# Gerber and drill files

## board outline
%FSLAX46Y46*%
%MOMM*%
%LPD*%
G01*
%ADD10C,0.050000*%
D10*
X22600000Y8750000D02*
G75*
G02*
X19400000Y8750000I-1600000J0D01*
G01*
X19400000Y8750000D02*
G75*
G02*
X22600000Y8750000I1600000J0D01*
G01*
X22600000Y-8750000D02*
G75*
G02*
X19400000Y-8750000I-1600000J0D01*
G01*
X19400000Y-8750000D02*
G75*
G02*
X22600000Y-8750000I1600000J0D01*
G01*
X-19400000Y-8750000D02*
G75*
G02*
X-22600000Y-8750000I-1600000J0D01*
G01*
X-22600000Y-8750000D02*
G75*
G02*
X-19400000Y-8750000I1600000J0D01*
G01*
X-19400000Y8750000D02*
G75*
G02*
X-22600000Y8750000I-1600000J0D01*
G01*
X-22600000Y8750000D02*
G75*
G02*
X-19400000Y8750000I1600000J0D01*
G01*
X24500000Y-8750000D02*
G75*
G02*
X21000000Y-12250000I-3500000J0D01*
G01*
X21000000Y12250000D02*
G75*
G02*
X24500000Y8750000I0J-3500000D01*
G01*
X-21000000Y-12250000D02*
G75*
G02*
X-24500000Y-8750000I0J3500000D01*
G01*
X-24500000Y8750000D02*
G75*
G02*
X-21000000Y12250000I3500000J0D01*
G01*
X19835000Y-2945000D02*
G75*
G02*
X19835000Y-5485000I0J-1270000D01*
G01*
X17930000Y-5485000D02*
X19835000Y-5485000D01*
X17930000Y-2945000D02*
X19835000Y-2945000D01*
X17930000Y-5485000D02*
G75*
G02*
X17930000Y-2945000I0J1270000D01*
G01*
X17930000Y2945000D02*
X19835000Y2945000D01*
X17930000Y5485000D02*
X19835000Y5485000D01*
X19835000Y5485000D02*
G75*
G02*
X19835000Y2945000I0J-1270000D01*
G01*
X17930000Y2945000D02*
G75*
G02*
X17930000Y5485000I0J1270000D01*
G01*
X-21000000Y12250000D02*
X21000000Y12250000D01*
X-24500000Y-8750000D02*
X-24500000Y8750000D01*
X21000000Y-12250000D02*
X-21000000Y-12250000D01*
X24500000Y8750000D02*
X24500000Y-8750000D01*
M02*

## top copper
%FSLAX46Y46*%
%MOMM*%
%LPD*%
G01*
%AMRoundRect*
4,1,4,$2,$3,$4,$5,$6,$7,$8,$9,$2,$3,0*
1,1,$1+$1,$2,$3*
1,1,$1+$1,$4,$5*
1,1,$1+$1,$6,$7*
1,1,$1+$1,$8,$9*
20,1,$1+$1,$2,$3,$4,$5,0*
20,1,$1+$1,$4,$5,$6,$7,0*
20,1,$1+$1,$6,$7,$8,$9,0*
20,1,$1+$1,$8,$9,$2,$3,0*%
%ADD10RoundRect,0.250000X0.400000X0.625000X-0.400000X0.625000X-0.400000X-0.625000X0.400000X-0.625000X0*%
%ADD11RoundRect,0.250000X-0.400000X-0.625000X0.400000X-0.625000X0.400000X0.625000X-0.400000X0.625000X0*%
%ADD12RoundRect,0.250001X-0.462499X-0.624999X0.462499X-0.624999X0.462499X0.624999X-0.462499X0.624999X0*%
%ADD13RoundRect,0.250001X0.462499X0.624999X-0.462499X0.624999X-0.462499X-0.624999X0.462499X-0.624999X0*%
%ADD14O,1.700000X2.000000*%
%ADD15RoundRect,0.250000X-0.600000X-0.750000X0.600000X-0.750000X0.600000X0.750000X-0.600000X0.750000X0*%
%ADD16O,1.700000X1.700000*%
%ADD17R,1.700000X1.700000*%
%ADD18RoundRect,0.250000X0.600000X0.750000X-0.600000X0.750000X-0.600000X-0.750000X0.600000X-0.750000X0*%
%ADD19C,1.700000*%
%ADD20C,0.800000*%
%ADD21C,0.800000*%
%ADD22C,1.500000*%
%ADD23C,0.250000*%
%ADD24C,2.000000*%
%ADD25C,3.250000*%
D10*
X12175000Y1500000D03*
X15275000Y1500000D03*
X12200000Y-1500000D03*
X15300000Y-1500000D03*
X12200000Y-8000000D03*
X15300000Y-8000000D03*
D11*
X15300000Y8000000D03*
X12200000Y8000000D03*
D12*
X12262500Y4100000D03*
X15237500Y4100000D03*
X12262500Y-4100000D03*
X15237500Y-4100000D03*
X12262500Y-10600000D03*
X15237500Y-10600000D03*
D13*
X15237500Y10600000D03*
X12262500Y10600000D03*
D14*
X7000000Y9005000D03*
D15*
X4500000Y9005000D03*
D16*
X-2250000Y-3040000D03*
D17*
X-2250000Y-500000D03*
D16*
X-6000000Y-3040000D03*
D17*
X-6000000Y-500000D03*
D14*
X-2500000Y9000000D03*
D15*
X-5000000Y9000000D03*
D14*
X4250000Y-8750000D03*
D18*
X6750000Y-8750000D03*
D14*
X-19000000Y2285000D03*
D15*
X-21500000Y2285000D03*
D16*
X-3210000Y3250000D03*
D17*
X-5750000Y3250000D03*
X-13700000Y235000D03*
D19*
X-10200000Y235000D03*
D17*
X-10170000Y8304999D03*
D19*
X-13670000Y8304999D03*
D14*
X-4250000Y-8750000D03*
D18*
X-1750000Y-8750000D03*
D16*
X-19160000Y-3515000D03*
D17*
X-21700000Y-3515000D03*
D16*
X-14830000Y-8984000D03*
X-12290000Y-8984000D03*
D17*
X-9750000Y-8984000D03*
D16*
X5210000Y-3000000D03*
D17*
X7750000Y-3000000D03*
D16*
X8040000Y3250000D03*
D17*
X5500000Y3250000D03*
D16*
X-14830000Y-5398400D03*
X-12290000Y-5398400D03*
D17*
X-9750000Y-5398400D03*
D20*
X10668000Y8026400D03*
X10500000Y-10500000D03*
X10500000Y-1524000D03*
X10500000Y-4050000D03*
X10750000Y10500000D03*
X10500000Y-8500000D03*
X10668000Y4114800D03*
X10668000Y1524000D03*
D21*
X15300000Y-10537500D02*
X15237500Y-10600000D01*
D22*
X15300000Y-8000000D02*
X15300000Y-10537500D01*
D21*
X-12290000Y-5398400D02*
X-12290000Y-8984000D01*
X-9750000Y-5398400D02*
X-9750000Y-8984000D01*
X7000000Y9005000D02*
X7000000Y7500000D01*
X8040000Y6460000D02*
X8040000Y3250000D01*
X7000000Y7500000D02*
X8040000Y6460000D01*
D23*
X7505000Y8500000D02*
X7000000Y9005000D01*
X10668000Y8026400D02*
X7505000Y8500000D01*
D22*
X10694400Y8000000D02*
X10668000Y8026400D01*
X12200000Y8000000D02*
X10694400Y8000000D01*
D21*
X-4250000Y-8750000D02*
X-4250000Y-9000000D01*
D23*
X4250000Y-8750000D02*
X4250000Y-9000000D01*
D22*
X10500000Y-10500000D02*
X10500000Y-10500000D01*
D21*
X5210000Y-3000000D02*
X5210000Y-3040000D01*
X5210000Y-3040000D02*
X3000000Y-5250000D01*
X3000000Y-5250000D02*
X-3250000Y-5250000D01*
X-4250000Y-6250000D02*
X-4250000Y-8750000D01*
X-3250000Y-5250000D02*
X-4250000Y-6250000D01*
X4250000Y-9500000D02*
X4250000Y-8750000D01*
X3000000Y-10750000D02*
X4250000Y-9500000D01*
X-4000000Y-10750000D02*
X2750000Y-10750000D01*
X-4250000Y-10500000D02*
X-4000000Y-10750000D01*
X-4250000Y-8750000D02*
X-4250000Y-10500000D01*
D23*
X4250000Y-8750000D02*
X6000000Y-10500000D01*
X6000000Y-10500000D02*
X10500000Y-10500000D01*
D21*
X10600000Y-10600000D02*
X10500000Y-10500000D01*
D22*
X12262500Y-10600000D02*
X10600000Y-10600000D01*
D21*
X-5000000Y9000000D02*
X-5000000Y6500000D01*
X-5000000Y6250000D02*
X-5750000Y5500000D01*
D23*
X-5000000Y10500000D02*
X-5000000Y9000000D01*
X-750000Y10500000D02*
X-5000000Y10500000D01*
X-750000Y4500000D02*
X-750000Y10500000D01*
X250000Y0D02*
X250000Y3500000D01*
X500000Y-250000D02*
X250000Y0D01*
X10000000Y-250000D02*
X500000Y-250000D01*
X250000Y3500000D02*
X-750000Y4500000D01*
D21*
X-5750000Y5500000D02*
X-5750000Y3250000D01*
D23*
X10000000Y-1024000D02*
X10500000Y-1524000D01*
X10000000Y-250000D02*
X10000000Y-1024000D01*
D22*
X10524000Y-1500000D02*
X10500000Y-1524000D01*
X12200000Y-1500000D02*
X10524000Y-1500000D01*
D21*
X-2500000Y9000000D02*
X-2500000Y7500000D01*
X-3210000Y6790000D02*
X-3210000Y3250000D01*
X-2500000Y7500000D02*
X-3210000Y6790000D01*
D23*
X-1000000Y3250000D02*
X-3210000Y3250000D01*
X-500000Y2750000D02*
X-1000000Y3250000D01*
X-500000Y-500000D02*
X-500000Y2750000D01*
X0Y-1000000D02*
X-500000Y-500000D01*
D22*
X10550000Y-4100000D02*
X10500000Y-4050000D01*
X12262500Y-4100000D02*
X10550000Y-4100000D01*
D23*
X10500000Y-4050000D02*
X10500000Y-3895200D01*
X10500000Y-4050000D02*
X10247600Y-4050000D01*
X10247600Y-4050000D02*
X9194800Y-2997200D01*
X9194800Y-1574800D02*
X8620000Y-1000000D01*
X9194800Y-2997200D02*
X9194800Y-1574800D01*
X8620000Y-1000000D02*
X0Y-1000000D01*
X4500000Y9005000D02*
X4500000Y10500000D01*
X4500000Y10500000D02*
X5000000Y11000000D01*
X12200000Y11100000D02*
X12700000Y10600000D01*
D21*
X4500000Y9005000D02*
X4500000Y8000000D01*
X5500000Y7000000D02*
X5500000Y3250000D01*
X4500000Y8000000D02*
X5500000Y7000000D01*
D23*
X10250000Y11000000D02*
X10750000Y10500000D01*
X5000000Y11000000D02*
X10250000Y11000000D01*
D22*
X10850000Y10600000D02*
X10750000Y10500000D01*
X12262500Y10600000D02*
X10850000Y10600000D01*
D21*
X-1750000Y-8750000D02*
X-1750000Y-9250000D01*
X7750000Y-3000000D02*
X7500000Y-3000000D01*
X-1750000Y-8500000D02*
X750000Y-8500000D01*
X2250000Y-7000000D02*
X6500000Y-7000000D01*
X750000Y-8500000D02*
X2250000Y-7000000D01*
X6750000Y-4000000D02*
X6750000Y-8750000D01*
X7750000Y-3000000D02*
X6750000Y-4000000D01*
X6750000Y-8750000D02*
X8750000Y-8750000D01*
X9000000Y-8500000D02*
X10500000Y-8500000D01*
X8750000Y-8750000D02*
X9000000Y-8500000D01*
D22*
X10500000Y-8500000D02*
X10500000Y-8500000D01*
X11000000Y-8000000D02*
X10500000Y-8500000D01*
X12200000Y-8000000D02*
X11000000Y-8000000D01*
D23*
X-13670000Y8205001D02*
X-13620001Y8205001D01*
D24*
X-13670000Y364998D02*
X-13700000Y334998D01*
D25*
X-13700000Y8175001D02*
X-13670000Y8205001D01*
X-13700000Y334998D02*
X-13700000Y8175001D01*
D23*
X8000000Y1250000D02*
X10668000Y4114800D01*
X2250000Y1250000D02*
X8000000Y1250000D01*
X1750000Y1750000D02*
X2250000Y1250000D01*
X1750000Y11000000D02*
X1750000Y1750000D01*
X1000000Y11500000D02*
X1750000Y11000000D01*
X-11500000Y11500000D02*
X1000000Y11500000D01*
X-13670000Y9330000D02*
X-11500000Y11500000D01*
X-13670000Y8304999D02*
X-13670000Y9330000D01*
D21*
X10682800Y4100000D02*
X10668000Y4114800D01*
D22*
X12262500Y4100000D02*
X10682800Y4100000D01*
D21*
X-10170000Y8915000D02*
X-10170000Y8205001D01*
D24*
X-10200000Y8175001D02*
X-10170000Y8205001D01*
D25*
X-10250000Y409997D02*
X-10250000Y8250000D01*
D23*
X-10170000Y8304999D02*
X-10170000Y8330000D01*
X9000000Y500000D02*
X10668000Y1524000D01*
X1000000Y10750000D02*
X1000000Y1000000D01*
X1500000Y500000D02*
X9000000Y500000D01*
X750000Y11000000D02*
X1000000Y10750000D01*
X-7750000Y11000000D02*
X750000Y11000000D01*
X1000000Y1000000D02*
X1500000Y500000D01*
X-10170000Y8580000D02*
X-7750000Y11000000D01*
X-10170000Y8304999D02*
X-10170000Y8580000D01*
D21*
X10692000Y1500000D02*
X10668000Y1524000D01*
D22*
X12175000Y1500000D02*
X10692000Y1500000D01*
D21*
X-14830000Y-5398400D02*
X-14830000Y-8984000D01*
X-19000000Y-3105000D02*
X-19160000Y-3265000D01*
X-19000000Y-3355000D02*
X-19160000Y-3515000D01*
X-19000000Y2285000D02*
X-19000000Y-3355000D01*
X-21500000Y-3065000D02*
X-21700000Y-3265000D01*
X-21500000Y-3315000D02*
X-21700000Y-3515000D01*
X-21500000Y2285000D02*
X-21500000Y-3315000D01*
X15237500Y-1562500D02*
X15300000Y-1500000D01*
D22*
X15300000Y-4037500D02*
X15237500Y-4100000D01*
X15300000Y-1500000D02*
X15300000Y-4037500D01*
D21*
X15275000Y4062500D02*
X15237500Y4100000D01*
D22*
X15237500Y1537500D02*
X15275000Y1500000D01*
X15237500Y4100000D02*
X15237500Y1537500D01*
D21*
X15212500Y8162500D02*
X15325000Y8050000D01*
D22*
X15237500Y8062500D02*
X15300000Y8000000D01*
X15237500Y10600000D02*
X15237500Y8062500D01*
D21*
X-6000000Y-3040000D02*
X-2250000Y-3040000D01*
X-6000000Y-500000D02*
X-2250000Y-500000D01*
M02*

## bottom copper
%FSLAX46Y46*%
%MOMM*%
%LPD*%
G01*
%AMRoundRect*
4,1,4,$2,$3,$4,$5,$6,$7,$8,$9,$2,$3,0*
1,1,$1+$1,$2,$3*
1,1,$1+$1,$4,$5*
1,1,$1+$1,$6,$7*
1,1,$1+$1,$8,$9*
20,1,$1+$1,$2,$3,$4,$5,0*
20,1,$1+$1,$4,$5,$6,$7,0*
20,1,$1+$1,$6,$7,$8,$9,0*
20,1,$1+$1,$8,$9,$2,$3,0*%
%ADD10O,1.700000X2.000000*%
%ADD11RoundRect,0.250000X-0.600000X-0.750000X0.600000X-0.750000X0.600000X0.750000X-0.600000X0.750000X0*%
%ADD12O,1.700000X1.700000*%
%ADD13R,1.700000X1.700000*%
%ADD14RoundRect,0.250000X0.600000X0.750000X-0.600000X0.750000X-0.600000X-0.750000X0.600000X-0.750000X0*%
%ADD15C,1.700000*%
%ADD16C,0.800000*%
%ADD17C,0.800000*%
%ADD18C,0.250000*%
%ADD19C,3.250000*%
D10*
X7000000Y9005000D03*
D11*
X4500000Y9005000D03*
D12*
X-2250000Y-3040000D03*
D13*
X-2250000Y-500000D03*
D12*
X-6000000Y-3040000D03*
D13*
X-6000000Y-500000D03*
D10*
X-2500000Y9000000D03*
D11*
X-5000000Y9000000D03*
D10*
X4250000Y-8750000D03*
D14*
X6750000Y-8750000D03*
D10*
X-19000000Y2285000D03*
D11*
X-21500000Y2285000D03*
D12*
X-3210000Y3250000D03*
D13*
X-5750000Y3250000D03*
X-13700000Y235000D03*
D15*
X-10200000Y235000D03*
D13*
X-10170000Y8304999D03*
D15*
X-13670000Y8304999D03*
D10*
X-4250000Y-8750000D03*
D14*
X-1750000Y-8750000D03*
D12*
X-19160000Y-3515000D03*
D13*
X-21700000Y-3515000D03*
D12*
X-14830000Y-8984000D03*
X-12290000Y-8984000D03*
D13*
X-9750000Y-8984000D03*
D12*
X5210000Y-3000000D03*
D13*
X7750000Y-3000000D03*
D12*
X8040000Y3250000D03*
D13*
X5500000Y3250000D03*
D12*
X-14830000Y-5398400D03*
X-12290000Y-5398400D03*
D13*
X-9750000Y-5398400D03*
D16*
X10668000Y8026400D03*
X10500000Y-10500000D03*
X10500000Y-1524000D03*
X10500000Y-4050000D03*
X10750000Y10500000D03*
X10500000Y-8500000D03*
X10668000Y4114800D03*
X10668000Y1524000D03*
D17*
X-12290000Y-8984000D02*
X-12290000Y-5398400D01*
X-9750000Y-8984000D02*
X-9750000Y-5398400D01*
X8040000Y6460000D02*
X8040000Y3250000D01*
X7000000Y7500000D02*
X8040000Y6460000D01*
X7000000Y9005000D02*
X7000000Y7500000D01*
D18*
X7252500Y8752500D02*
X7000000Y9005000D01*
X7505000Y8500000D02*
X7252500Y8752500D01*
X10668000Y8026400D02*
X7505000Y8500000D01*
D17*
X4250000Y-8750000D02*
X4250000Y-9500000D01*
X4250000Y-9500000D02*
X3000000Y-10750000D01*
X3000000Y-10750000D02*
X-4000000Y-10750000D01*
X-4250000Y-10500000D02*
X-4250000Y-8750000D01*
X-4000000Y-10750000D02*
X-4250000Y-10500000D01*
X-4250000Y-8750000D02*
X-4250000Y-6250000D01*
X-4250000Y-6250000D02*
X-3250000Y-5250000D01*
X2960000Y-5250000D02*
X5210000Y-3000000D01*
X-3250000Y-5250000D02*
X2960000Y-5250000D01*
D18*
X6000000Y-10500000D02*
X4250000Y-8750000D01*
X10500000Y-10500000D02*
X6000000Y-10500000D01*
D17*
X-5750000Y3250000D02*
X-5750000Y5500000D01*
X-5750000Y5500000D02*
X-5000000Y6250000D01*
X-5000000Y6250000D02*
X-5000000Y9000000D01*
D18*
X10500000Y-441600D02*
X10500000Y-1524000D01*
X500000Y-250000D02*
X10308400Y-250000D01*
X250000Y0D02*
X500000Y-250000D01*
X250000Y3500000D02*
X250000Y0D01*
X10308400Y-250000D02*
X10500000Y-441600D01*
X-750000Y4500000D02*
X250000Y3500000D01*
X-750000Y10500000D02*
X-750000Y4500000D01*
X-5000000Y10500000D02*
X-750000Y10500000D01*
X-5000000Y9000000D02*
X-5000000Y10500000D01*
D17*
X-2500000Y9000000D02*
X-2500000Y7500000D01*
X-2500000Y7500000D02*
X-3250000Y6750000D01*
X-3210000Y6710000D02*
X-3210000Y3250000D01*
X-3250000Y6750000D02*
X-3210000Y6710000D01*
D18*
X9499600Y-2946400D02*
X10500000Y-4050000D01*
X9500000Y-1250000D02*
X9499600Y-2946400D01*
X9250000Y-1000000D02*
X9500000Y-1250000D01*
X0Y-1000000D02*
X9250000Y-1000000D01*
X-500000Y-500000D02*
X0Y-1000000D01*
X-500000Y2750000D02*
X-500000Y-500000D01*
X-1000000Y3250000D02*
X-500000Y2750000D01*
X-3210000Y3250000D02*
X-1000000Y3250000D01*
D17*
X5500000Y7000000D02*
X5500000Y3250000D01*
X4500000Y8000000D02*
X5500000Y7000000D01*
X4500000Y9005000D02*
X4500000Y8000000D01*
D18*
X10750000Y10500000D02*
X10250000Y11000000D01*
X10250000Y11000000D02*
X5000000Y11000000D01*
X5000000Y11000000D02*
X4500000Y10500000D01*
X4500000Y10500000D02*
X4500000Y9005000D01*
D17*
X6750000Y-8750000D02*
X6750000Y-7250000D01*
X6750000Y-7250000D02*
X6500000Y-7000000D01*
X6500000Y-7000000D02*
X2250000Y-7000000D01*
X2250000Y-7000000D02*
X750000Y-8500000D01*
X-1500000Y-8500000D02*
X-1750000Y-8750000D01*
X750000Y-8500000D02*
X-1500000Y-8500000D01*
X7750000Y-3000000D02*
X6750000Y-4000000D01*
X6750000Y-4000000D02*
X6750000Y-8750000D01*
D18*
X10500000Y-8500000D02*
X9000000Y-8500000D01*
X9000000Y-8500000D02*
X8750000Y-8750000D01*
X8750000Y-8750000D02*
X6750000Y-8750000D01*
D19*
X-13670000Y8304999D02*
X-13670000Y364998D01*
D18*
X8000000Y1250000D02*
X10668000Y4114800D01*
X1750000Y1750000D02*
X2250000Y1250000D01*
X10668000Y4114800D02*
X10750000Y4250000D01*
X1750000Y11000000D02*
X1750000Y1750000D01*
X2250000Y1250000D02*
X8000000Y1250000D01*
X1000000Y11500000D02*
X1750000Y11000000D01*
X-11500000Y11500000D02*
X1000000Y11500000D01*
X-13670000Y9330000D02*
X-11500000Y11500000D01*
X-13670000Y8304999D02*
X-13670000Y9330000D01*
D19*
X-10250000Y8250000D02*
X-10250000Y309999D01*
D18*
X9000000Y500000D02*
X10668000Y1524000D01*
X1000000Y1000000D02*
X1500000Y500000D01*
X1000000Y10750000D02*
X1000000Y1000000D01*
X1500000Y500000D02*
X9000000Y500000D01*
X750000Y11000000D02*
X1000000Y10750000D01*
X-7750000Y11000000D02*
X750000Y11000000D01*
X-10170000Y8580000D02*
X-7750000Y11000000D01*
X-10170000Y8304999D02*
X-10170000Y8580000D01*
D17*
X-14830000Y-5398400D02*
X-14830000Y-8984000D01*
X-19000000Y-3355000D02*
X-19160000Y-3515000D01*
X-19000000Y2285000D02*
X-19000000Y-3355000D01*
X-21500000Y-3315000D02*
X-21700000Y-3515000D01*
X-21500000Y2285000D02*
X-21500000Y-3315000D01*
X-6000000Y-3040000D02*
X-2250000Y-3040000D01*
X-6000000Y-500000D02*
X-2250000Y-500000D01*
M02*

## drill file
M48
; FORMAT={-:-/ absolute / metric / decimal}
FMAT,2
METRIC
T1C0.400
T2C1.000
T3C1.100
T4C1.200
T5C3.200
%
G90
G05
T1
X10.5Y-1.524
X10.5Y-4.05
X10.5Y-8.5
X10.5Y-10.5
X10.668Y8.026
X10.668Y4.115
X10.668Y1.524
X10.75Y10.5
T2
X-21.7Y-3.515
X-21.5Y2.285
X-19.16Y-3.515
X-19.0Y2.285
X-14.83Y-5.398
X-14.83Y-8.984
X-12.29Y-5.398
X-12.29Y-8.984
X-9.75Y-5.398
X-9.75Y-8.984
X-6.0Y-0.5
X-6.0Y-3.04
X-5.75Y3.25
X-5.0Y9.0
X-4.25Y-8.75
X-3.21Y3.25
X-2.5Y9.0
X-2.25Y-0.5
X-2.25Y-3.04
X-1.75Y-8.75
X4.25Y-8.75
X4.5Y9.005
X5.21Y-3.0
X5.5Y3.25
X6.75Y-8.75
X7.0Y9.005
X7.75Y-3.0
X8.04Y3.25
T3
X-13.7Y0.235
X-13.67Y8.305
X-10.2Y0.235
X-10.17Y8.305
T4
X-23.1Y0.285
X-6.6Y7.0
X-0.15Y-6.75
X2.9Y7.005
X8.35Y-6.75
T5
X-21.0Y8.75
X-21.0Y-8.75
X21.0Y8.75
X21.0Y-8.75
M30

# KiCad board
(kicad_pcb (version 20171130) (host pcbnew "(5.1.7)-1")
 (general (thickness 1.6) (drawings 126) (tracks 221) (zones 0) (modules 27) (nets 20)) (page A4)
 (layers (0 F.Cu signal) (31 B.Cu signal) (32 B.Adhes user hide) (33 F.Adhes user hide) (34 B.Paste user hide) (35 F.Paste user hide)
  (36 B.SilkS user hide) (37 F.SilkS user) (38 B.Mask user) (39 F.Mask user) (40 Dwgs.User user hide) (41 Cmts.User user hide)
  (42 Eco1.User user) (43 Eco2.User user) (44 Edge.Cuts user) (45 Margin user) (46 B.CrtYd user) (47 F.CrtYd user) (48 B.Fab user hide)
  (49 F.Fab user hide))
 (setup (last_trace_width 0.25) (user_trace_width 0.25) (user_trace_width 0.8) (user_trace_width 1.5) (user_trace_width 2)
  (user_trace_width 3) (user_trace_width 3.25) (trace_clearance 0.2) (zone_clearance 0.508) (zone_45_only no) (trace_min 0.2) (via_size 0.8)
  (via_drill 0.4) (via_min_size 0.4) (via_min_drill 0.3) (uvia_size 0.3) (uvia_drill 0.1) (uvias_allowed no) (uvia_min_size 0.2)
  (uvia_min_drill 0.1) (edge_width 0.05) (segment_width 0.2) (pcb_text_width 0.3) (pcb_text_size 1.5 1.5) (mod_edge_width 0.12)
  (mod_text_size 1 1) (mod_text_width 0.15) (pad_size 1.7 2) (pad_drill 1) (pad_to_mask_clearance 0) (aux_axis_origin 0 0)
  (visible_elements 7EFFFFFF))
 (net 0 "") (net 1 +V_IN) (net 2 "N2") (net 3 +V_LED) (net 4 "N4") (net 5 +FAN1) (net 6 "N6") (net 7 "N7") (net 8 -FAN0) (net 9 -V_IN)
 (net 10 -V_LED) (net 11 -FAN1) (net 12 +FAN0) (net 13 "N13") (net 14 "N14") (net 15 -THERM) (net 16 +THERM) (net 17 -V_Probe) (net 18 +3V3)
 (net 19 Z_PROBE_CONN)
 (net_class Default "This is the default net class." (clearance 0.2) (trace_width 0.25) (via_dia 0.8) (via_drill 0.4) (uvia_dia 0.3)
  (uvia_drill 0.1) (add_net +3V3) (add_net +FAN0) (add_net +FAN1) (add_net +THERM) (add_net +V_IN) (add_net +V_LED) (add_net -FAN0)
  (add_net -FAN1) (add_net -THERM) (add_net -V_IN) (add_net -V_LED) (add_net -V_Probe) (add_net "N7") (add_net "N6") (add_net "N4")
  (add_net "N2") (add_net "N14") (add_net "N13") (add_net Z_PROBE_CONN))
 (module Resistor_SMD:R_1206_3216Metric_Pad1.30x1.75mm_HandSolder (layer F.Cu) (at 13.725 -1.5 180)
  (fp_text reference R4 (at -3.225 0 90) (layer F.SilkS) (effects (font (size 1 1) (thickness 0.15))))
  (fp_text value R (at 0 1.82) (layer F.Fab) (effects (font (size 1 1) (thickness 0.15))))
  (pad 2 smd roundrect (at 1.55 0 180) (size 1.3 1.75) (layers F.Cu F.Paste F.Mask) (roundrect_rratio 0.192308) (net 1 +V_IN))
  (pad 1 smd roundrect (at -1.55 0 180) (size 1.3 1.75) (layers F.Cu F.Paste F.Mask) (roundrect_rratio 0.192308) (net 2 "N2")))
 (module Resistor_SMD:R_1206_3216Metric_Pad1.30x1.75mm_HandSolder (layer F.Cu) (at 13.75 1.5 180)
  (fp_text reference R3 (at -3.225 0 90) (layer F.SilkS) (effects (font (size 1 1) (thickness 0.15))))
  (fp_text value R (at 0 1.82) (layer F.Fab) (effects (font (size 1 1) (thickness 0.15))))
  (pad 2 smd roundrect (at 1.55 0 180) (size 1.3 1.75) (layers F.Cu F.Paste F.Mask) (roundrect_rratio 0.192308) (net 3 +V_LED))
  (pad 1 smd roundrect (at -1.55 0 180) (size 1.3 1.75) (layers F.Cu F.Paste F.Mask) (roundrect_rratio 0.192308) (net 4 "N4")))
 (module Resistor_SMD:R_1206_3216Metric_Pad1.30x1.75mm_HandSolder (layer F.Cu) (at 13.75 8 180)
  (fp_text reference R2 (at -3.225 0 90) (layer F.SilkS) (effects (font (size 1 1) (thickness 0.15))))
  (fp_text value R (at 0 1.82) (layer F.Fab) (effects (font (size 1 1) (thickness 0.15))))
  (pad 2 smd roundrect (at 1.55 0 180) (size 1.3 1.75) (layers F.Cu F.Paste F.Mask) (roundrect_rratio 0.192308) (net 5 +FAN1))
  (pad 1 smd roundrect (at -1.55 0 180) (size 1.3 1.75) (layers F.Cu F.Paste F.Mask) (roundrect_rratio 0.192308) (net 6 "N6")))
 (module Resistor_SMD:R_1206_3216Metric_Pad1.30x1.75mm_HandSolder (layer F.Cu) (at 13.75 -8)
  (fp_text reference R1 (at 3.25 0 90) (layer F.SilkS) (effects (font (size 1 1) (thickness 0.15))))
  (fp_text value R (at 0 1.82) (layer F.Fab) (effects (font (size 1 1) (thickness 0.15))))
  (pad 2 smd roundrect (at 1.55 0) (size 1.3 1.75) (layers F.Cu F.Paste F.Mask) (roundrect_rratio 0.192308) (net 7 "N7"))
  (pad 1 smd roundrect (at -1.55 0) (size 1.3 1.75) (layers F.Cu F.Paste F.Mask) (roundrect_rratio 0.192308) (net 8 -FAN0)))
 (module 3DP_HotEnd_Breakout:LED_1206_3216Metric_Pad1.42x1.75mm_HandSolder (layer F.Cu) (at 13.75 -4.1)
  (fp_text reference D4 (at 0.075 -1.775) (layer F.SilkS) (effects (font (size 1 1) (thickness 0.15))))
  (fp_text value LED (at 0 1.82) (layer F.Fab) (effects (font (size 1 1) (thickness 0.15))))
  (pad 1 smd roundrect (at -1.4875 0) (size 1.425 1.75) (layers F.Cu F.Paste F.Mask) (roundrect_rratio 0.175439) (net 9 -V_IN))
  (pad 2 smd roundrect (at 1.4875 0) (size 1.425 1.75) (layers F.Cu F.Paste F.Mask) (roundrect_rratio 0.175439) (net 2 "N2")))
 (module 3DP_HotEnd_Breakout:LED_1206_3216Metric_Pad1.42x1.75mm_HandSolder (layer F.Cu) (at 13.75 4.1)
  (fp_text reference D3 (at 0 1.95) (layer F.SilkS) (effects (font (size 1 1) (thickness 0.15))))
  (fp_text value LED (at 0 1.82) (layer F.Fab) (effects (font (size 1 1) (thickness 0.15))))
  (pad 1 smd roundrect (at -1.4875 0) (size 1.425 1.75) (layers F.Cu F.Paste F.Mask) (roundrect_rratio 0.175439) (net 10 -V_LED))
  (pad 2 smd roundrect (at 1.4875 0) (size 1.425 1.75) (layers F.Cu F.Paste F.Mask) (roundrect_rratio 0.175439) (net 4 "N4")))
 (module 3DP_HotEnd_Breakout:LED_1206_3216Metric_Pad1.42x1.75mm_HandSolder (layer F.Cu) (at 13.75 10.6)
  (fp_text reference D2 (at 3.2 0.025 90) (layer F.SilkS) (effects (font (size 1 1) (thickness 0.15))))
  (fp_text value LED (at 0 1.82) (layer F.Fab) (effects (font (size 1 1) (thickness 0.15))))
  (pad 1 smd roundrect (at -1.4875 0) (size 1.425 1.75) (layers F.Cu F.Paste F.Mask) (roundrect_rratio 0.175439) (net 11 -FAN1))
  (pad 2 smd roundrect (at 1.4875 0) (size 1.425 1.75) (layers F.Cu F.Paste F.Mask) (roundrect_rratio 0.175439) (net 6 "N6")))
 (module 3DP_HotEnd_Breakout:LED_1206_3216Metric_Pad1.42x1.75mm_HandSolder (layer F.Cu) (at 13.75 -10.6 180)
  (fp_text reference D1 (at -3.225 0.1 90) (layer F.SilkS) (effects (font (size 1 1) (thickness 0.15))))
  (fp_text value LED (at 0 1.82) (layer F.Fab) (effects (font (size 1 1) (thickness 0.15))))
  (pad 1 smd roundrect (at -1.4875 0 180) (size 1.425 1.75) (layers F.Cu F.Paste F.Mask) (roundrect_rratio 0.175439) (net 7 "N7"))
  (pad 2 smd roundrect (at 1.4875 0 180) (size 1.425 1.75) (layers F.Cu F.Paste F.Mask) (roundrect_rratio 0.175439) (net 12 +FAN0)))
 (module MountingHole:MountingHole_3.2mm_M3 (layer F.Cu) (at -21 8.75)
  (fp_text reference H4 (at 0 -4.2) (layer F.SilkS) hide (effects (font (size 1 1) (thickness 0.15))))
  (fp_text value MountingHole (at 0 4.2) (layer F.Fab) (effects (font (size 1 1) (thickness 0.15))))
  (pad 1 np_thru_hole circle (at 0 0) (size 3.2 3.2) (drill 3.2) (layers *.Cu *.Mask)))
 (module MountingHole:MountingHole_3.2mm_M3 (layer F.Cu) (at 21 -8.75)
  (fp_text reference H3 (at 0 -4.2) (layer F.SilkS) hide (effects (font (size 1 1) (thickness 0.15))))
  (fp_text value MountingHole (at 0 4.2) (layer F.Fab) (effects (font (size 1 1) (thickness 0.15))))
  (pad 1 np_thru_hole circle (at 0 0) (size 3.2 3.2) (drill 3.2) (layers *.Cu *.Mask)))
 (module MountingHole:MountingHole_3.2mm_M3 (layer F.Cu) (at 21 8.75)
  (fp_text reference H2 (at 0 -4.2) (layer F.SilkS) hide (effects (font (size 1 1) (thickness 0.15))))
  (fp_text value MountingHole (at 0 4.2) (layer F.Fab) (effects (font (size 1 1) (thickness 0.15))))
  (pad 1 np_thru_hole circle (at 0 0) (size 3.2 3.2) (drill 3.2) (layers *.Cu *.Mask)))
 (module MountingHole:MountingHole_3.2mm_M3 (layer F.Cu) (at -21 -8.75)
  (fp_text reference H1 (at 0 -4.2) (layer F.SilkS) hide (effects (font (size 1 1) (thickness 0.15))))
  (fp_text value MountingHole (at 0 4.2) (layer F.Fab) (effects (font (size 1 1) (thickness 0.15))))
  (pad 1 np_thru_hole circle (at 0 0) (size 3.2 3.2) (drill 3.2) (layers *.Cu *.Mask)))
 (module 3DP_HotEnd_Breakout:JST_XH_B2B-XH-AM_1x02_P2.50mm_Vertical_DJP (layer F.Cu) (at 4.5 -9.005)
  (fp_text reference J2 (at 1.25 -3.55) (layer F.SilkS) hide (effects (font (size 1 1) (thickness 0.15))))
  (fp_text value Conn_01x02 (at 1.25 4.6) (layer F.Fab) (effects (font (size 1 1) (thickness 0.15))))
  (pad "" np_thru_hole circle (at -1.6 2) (size 1.2 1.2) (drill 1.2) (layers *.Cu *.Mask))
  (pad 2 thru_hole oval (at 2.5 0) (size 1.7 2) (drill 1) (layers *.Cu *.Mask) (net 8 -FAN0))
  (pad 1 thru_hole roundrect (at 0 0) (size 1.7 2) (drill 1) (layers *.Cu *.Mask) (roundrect_rratio 0.147059) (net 12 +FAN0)))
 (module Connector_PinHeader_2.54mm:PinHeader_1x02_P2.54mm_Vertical (layer F.Cu) (at -2.25 0.5)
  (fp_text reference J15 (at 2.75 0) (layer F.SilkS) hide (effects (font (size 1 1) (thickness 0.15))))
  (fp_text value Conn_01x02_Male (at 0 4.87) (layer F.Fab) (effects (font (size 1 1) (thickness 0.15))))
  (pad 2 thru_hole oval (at 0 2.54) (size 1.7 1.7) (drill 1) (layers *.Cu *.Mask) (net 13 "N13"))
  (pad 1 thru_hole rect (at 0 0) (size 1.7 1.7) (drill 1) (layers *.Cu *.Mask) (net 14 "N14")))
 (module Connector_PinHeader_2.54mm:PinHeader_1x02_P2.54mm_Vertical (layer F.Cu) (at -6 0.5)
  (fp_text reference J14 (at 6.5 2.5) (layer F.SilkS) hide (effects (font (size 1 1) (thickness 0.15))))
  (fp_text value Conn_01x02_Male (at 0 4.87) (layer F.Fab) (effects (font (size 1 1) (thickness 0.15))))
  (pad 2 thru_hole oval (at 0 2.54) (size 1.7 1.7) (drill 1) (layers *.Cu *.Mask) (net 13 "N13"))
  (pad 1 thru_hole rect (at 0 0) (size 1.7 1.7) (drill 1) (layers *.Cu *.Mask) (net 14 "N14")))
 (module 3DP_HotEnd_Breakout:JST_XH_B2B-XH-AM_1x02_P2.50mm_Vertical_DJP (layer F.Cu) (at -5 -9)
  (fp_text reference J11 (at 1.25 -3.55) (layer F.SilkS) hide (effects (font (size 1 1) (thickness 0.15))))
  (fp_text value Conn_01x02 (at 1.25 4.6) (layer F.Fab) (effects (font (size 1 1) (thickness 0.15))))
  (pad "" np_thru_hole circle (at -1.6 2) (size 1.2 1.2) (drill 1.2) (layers *.Cu *.Mask))
  (pad 2 thru_hole oval (at 2.5 0) (size 1.7 2) (drill 1) (layers *.Cu *.Mask) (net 10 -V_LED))
  (pad 1 thru_hole roundrect (at 0 0) (size 1.7 2) (drill 1) (layers *.Cu *.Mask) (roundrect_rratio 0.147059) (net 3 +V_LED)))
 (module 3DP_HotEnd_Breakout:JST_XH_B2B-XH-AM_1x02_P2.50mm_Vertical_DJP (layer F.Cu) (at 6.75 8.75 180)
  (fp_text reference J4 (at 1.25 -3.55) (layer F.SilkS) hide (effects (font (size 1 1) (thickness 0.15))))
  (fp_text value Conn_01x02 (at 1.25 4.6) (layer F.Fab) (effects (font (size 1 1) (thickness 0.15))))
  (pad "" np_thru_hole circle (at -1.6 2 180) (size 1.2 1.2) (drill 1.2) (layers *.Cu *.Mask))
  (pad 2 thru_hole oval (at 2.5 0 180) (size 1.7 2) (drill 1) (layers *.Cu *.Mask) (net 11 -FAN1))
  (pad 1 thru_hole roundrect (at 0 0 180) (size 1.7 2) (drill 1) (layers *.Cu *.Mask) (roundrect_rratio 0.147059) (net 5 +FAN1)))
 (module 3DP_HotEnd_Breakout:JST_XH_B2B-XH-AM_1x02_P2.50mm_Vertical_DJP (layer F.Cu) (at -21.5 -2.285)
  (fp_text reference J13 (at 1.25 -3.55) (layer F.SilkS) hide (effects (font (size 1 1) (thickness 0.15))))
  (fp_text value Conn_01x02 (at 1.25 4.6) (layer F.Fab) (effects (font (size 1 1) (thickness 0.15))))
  (pad "" np_thru_hole circle (at -1.6 2) (size 1.2 1.2) (drill 1.2) (layers *.Cu *.Mask))
  (pad 2 thru_hole oval (at 2.5 0) (size 1.7 2) (drill 1) (layers *.Cu *.Mask) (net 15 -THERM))
  (pad 1 thru_hole roundrect (at 0 0) (size 1.7 2) (drill 1) (layers *.Cu *.Mask) (roundrect_rratio 0.147059) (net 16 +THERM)))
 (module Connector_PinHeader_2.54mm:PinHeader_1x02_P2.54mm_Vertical (layer F.Cu) (at -5.75 -3.25 90)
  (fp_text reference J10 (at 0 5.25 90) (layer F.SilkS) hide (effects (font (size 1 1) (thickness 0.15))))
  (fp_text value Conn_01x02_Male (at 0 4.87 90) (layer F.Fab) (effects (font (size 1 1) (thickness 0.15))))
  (pad 2 thru_hole oval (at 0 2.54 90) (size 1.7 1.7) (drill 1) (layers *.Cu *.Mask) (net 10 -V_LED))
  (pad 1 thru_hole rect (at 0 0 90) (size 1.7 1.7) (drill 1) (layers *.Cu *.Mask) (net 3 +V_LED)))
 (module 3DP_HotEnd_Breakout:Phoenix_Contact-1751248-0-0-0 (layer F.Cu) (at -11.95 -0.284999)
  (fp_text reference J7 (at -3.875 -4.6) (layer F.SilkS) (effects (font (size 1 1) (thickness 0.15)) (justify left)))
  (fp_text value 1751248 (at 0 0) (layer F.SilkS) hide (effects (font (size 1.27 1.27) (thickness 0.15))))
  (pad 1 thru_hole rect (at -1.75 0.049999) (size 1.7 1.7) (drill 1.1) (layers *.Cu) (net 1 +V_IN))
  (pad 2 thru_hole circle (at 1.75 0.049999) (size 1.7 1.7) (drill 1.1) (layers *.Cu) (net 9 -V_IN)))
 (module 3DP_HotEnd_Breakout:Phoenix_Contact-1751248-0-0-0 (layer F.Cu) (at -11.92 -8.255 180)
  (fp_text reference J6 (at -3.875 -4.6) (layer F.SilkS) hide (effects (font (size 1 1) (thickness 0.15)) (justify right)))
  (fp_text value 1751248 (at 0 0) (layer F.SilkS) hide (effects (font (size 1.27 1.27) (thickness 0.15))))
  (pad 1 thru_hole rect (at -1.75 0.049999 180) (size 1.7 1.7) (drill 1.1) (layers *.Cu) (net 1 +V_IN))
  (pad 2 thru_hole circle (at 1.75 0.049999 180) (size 1.7 1.7) (drill 1.1) (layers *.Cu) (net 9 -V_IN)))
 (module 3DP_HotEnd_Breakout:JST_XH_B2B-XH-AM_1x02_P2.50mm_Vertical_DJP (layer F.Cu) (at -1.75 8.75 180)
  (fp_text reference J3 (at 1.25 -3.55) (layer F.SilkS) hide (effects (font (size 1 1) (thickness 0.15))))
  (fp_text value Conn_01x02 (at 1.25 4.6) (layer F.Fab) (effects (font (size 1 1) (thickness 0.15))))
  (pad "" np_thru_hole circle (at -1.6 2 180) (size 1.2 1.2) (drill 1.2) (layers *.Cu *.Mask))
  (pad 2 thru_hole oval (at 2.5 0 180) (size 1.7 2) (drill 1) (layers *.Cu *.Mask) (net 11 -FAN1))
  (pad 1 thru_hole roundrect (at 0 0 180) (size 1.7 2) (drill 1) (layers *.Cu *.Mask) (roundrect_rratio 0.147059) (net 5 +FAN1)))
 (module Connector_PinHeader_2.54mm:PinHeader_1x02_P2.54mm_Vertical (layer F.Cu) (at -21.7 3.515 90)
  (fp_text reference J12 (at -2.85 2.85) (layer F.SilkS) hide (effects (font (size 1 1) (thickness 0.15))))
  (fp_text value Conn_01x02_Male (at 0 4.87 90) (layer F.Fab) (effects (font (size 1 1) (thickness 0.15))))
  (pad 2 thru_hole oval (at 0 2.54 90) (size 1.7 1.7) (drill 1) (layers *.Cu *.Mask) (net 15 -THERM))
  (pad 1 thru_hole rect (at 0 0 90) (size 1.7 1.7) (drill 1) (layers *.Cu *.Mask) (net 16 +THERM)))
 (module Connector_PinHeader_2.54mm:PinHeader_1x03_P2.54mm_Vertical (layer F.Cu) (at -9.75 8.984 270)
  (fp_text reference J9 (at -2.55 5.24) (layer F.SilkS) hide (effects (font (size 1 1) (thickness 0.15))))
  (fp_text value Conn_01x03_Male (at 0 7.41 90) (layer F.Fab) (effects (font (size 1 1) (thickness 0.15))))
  (pad 3 thru_hole oval (at 0 5.08 270) (size 1.7 1.7) (drill 1) (layers *.Cu *.Mask) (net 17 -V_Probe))
  (pad 2 thru_hole oval (at 0 2.54 270) (size 1.7 1.7) (drill 1) (layers *.Cu *.Mask) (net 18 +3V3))
  (pad 1 thru_hole rect (at 0 0 270) (size 1.7 1.7) (drill 1) (layers *.Cu *.Mask) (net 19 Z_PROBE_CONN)))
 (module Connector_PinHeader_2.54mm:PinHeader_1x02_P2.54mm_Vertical (layer F.Cu) (at 7.75 3 270)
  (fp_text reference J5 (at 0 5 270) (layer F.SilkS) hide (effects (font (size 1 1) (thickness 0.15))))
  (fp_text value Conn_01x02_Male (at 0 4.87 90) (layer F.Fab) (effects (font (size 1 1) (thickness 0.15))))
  (pad 2 thru_hole oval (at 0 2.54 270) (size 1.7 1.7) (drill 1) (layers *.Cu *.Mask) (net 11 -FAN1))
  (pad 1 thru_hole rect (at 0 0 270) (size 1.7 1.7) (drill 1) (layers *.Cu *.Mask) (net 5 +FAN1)))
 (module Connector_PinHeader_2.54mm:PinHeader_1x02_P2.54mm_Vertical (layer F.Cu) (at 5.5 -3.25 90)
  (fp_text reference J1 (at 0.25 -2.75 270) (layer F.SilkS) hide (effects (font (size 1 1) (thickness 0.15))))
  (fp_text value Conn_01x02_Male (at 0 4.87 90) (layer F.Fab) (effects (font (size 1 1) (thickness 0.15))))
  (pad 2 thru_hole oval (at 0 2.54 90) (size 1.7 1.7) (drill 1) (layers *.Cu *.Mask) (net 8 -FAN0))
  (pad 1 thru_hole rect (at 0 0 90) (size 1.7 1.7) (drill 1) (layers *.Cu *.Mask) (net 12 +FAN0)))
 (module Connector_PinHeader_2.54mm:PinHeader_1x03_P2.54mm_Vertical (layer F.Cu) (at -9.75 5.3984 270)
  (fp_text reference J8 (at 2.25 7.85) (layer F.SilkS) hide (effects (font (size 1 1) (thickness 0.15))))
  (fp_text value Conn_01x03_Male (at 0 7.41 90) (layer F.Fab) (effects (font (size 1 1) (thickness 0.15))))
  (pad 3 thru_hole oval (at 0 5.08 270) (size 1.7 1.7) (drill 1) (layers *.Cu *.Mask) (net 17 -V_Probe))
  (pad 2 thru_hole oval (at 0 2.54 270) (size 1.7 1.7) (drill 1) (layers *.Cu *.Mask) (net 18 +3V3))
  (pad 1 thru_hole rect (at 0 0 270) (size 1.7 1.7) (drill 1) (layers *.Cu *.Mask) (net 19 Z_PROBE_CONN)))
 (gr_circle (center 21 -8.75) (end 22.6 -8.75) (layer Edge.Cuts) (width 0.05))
 (gr_circle (center 21 8.75) (end 22.6 8.75) (layer Edge.Cuts) (width 0.05))
 (gr_circle (center -21 8.75) (end -19.4 8.75) (layer Edge.Cuts) (width 0.05))
 (gr_circle (center -21 -8.75) (end -19.4 -8.75) (layer Edge.Cuts) (width 0.05))
 (gr_arc (start 21 8.75) (end 21 12.25) (angle -90) (layer Edge.Cuts) (width 0.05))
 (gr_arc (start 21 -8.75) (end 24.5 -8.75) (angle -90) (layer Edge.Cuts) (width 0.05))
 (gr_arc (start -21 8.75) (end -24.5 8.75) (angle -90) (layer Edge.Cuts) (width 0.05))
 (gr_arc (start -21 -8.75) (end -21 -12.25) (angle -90) (layer Edge.Cuts) (width 0.05))
 (gr_arc (start 19.835 4.215) (end 19.835 5.485) (angle -180) (layer Edge.Cuts) (width 0.05))
 (gr_line (start 17.93 5.485) (end 19.835 5.485) (layer Edge.Cuts) (width 0.05))
 (gr_line (start 17.93 2.945) (end 19.835 2.945) (layer Edge.Cuts) (width 0.05))
 (gr_arc (start 17.93 4.215) (end 17.93 2.945) (angle -180) (layer Edge.Cuts) (width 0.05))
 (gr_line (start 17.93 -2.945) (end 19.835 -2.945) (layer Edge.Cuts) (width 0.05))
 (gr_line (start 17.93 -5.485) (end 19.835 -5.485) (layer Edge.Cuts) (width 0.05))
 (gr_arc (start 19.835 -4.215) (end 19.835 -2.945) (angle -180) (layer Edge.Cuts) (width 0.05))
 (gr_arc (start 17.93 -4.215) (end 17.93 -5.485) (angle -180) (layer Edge.Cuts) (width 0.05))
 (gr_line (start -21 -12.25) (end 21 -12.25) (layer Edge.Cuts) (width 0.05))
 (gr_line (start -24.5 8.75) (end -24.5 -8.75) (layer Edge.Cuts) (width 0.05))
 (gr_line (start 21 12.25) (end -21 12.25) (layer Edge.Cuts) (width 0.05))
 (gr_line (start 24.5 -8.75) (end 24.5 8.75) (layer Edge.Cuts) (width 0.05))
 (segment (start 15.3 10.5375) (end 15.2375 10.6) (width 0.8) (layer F.Cu) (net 6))
 (segment (start 15.3 8) (end 15.3 10.5375) (width 1.5) (layer F.Cu) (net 6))
 (segment (start -12.29 8.984) (end -12.29 5.3984) (width 0.8) (layer B.Cu) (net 18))
 (segment (start -12.29 5.3984) (end -12.29 8.984) (width 0.8) (layer F.Cu) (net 18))
 (segment (start -9.75 8.984) (end -9.75 5.3984) (width 0.8) (layer B.Cu) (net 19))
 (segment (start -9.75 5.3984) (end -9.75 8.984) (width 0.8) (layer F.Cu) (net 19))
 (segment (start 7 -9.005) (end 7 -7.5) (width 0.8) (layer F.Cu) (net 8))
 (segment (start 8.04 -6.46) (end 8.04 -3.25) (width 0.8) (layer F.Cu) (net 8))
 (segment (start 7 -7.5) (end 8.04 -6.46) (width 0.8) (layer F.Cu) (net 8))
 (via (at 10.668 -8.0264) (size 0.8) (drill 0.4) (layers F.Cu B.Cu) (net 8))
 (segment (start 8.04 -6.46) (end 8.04 -3.25) (width 0.8) (layer B.Cu) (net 8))
 (segment (start 7 -7.5) (end 8.04 -6.46) (width 0.8) (layer B.Cu) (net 8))
 (segment (start 7 -9.005) (end 7 -7.5) (width 0.8) (layer B.Cu) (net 8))
 (segment (start 7.505 -8.5) (end 7 -9.005) (width 0.25) (layer F.Cu) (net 8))
 (segment (start 10.668 -8.0264) (end 7.505 -8.5) (width 0.25) (layer F.Cu) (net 8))
 (segment (start 10.6944 -8) (end 10.668 -8.0264) (width 1.5) (layer F.Cu) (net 8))
 (segment (start 12.2 -8) (end 10.6944 -8) (width 1.5) (layer F.Cu) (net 8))
 (segment (start 7.2525 -8.7525) (end 7 -9.005) (width 0.25) (layer B.Cu) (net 8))
 (segment (start 7.505 -8.5) (end 7.2525 -8.7525) (width 0.25) (layer B.Cu) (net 8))
 (segment (start 10.668 -8.0264) (end 7.505 -8.5) (width 0.25) (layer B.Cu) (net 8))
 (segment (start -4.25 8.75) (end -4.25 9) (width 0.8) (layer F.Cu) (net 11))
 (segment (start 4.25 8.75) (end 4.25 9) (width 0.25) (layer F.Cu) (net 11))
 (segment (start 10.5 10.5) (end 10.5 10.5) (width 1.5) (layer F.Cu) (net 11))
 (via (at 10.5 10.5) (size 0.8) (drill 0.4) (layers F.Cu B.Cu) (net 11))
 (segment (start 4.25 8.75) (end 4.25 9.5) (width 0.8) (layer B.Cu) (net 11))
 (segment (start 4.25 9.5) (end 3 10.75) (width 0.8) (layer B.Cu) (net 11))
 (segment (start 3 10.75) (end -4 10.75) (width 0.8) (layer B.Cu) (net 11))
 (segment (start -4.25 10.5) (end -4.25 8.75) (width 0.8) (layer B.Cu) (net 11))
 (segment (start -4 10.75) (end -4.25 10.5) (width 0.8) (layer B.Cu) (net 11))
 (segment (start -4.25 8.75) (end -4.25 6.25) (width 0.8) (layer B.Cu) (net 11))
 (segment (start -4.25 6.25) (end -3.25 5.25) (width 0.8) (layer B.Cu) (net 11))
 (segment (start 2.96 5.25) (end 5.21 3) (width 0.8) (layer B.Cu) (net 11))
 (segment (start -3.25 5.25) (end 2.96 5.25) (width 0.8) (layer B.Cu) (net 11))
 (segment (start 6 10.5) (end 4.25 8.75) (width 0.25) (layer B.Cu) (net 11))
 (segment (start 10.5 10.5) (end 6 10.5) (width 0.25) (layer B.Cu) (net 11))
 (segment (start 5.21 3) (end 5.21 3.04) (width 0.8) (layer F.Cu) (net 11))
 (segment (start 5.21 3.04) (end 3 5.25) (width 0.8) (layer F.Cu) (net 11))
 (segment (start 3 5.25) (end -3.25 5.25) (width 0.8) (layer F.Cu) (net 11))
 (segment (start -4.25 6.25) (end -4.25 8.75) (width 0.8) (layer F.Cu) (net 11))
 (segment (start -3.25 5.25) (end -4.25 6.25) (width 0.8) (layer F.Cu) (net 11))
 (segment (start 4.25 9.5) (end 4.25 8.75) (width 0.8) (layer F.Cu) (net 11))
 (segment (start 3 10.75) (end 4.25 9.5) (width 0.8) (layer F.Cu) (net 11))
 (segment (start -4 10.75) (end 2.75 10.75) (width 0.8) (layer F.Cu) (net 11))
 (segment (start -4.25 10.5) (end -4 10.75) (width 0.8) (layer F.Cu) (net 11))
 (segment (start -4.25 8.75) (end -4.25 10.5) (width 0.8) (layer F.Cu) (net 11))
 (segment (start 4.25 8.75) (end 6 10.5) (width 0.25) (layer F.Cu) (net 11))
 (segment (start 6 10.5) (end 10.5 10.5) (width 0.25) (layer F.Cu) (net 11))
 (segment (start 10.6 10.6) (end 10.5 10.5) (width 0.8) (layer F.Cu) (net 11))
 (segment (start 12.2625 10.6) (end 10.6 10.6) (width 1.5) (layer F.Cu) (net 11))
 (segment (start -5 -9) (end -5 -6.5) (width 0.8) (layer F.Cu) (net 3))
 (segment (start -5 -6.25) (end -5.75 -5.5) (width 0.8) (layer F.Cu) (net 3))
 (segment (start -5 -10.5) (end -5 -9) (width 0.25) (layer F.Cu) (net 3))
 (segment (start -0.75 -10.5) (end -5 -10.5) (width 0.25) (layer F.Cu) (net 3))
 (segment (start -0.75 -4.5) (end -0.75 -10.5) (width 0.25) (layer F.Cu) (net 3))
 (segment (start 0.25 0) (end 0.25 -3.5) (width 0.25) (layer F.Cu) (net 3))
 (segment (start 0.5 0.25) (end 0.25 0) (width 0.25) (layer F.Cu) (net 3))
 (segment (start 10 0.25) (end 0.5 0.25) (width 0.25) (layer F.Cu) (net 3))
 (segment (start 0.25 -3.5) (end -0.75 -4.5) (width 0.25) (layer F.Cu) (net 3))
 (via (at 10.5 1.524) (size 0.8) (drill 0.4) (layers F.Cu B.Cu) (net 3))
 (segment (start -5.75 -3.25) (end -5.75 -5.5) (width 0.8) (layer B.Cu) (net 3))
 (segment (start -5.75 -5.5) (end -5 -6.25) (width 0.8) (layer B.Cu) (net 3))
 (segment (start -5 -6.25) (end -5 -9) (width 0.8) (layer B.Cu) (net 3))
 (segment (start -5.75 -5.5) (end -5.75 -3.25) (width 0.8) (layer F.Cu) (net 3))
 (segment (start 10 1.024) (end 10.5 1.524) (width 0.25) (layer F.Cu) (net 3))
 (segment (start 10 0.25) (end 10 1.024) (width 0.25) (layer F.Cu) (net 3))
 (segment (start 10.524 1.5) (end 10.5 1.524) (width 1.5) (layer F.Cu) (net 3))
 (segment (start 12.2 1.5) (end 10.524 1.5) (width 1.5) (layer F.Cu) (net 3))
 (segment (start 10.5 0.4416) (end 10.5 1.524) (width 0.25) (layer B.Cu) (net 3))
 (segment (start 0.5 0.25) (end 10.3084 0.25) (width 0.25) (layer B.Cu) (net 3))
 (segment (start 0.25 0) (end 0.5 0.25) (width 0.25) (layer B.Cu) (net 3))
 (segment (start 0.25 -3.5) (end 0.25 0) (width 0.25) (layer B.Cu) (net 3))
 (segment (start 10.3084 0.25) (end 10.5 0.4416) (width 0.25) (layer B.Cu) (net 3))
 (segment (start -0.75 -4.5) (end 0.25 -3.5) (width 0.25) (layer B.Cu) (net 3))
 (segment (start -0.75 -10.5) (end -0.75 -4.5) (width 0.25) (layer B.Cu) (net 3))
 (segment (start -5 -10.5) (end -0.75 -10.5) (width 0.25) (layer B.Cu) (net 3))
 (segment (start -5 -9) (end -5 -10.5) (width 0.25) (layer B.Cu) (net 3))
 (segment (start -2.5 -9) (end -2.5 -7.5) (width 0.8) (layer F.Cu) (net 10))
 (segment (start -3.21 -6.79) (end -3.21 -3.25) (width 0.8) (layer F.Cu) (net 10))
 (segment (start -2.5 -7.5) (end -3.21 -6.79) (width 0.8) (layer F.Cu) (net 10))
 (segment (start -1 -3.25) (end -3.21 -3.25) (width 0.25) (layer F.Cu) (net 10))
 (segment (start -0.5 -2.75) (end -1 -3.25) (width 0.25) (layer F.Cu) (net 10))
 (segment (start -0.5 0.5) (end -0.5 -2.75) (width 0.25) (layer F.Cu) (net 10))
 (segment (start 0 1) (end -0.5 0.5) (width 0.25) (layer F.Cu) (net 10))
 (via (at 10.5 4.05) (size 0.8) (drill 0.4) (layers F.Cu B.Cu) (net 10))
 (segment (start -2.5 -9) (end -2.5 -7.5) (width 0.8) (layer B.Cu) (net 10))
 (segment (start -2.5 -7.5) (end -3.25 -6.75) (width 0.8) (layer B.Cu) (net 10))
 (segment (start -3.21 -6.71) (end -3.21 -3.25) (width 0.8) (layer B.Cu) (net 10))
 (segment (start -3.25 -6.75) (end -3.21 -6.71) (width 0.8) (layer B.Cu) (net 10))
 (segment (start 10.55 4.1) (end 10.5 4.05) (width 1.5) (layer F.Cu) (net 10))
 (segment (start 12.2625 4.1) (end 10.55 4.1) (width 1.5) (layer F.Cu) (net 10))
 (segment (start 10.5 4.05) (end 10.5 3.8952) (width 0.25) (layer F.Cu) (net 10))
 (segment (start 10.5 4.05) (end 10.2476 4.05) (width 0.25) (layer F.Cu) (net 10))
 (segment (start 10.2476 4.05) (end 9.1948 2.9972) (width 0.25) (layer F.Cu) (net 10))
 (segment (start 9.1948 1.5748) (end 8.62 1) (width 0.25) (layer F.Cu) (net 10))
 (segment (start 9.1948 2.9972) (end 9.1948 1.5748) (width 0.25) (layer F.Cu) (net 10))
 (segment (start 8.62 1) (end 0 1) (width 0.25) (layer F.Cu) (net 10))
 (segment (start 9.4996 2.9464) (end 10.5 4.05) (width 0.25) (layer B.Cu) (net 10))
 (segment (start 9.5 1.25) (end 9.4996 2.9464) (width 0.25) (layer B.Cu) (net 10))
 (segment (start 9.25 1) (end 9.5 1.25) (width 0.25) (layer B.Cu) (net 10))
 (segment (start 0 1) (end 9.25 1) (width 0.25) (layer B.Cu) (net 10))
 (segment (start -0.5 0.5) (end 0 1) (width 0.25) (layer B.Cu) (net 10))
 (segment (start -0.5 -2.75) (end -0.5 0.5) (width 0.25) (layer B.Cu) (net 10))
 (segment (start -1 -3.25) (end -0.5 -2.75) (width 0.25) (layer B.Cu) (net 10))
 (segment (start -3.21 -3.25) (end -1 -3.25) (width 0.25) (layer B.Cu) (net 10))
 (segment (start 4.5 -9.005) (end 4.5 -10.5) (width 0.25) (layer F.Cu) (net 12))
 (segment (start 4.5 -10.5) (end 5 -11) (width 0.25) (layer F.Cu) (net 12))
 (segment (start 12.2 -11.1) (end 12.7 -10.6) (width 0.25) (layer F.Cu) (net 12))
 (segment (start 4.5 -9.005) (end 4.5 -8) (width 0.8) (layer F.Cu) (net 12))
 (segment (start 5.5 -7) (end 5.5 -3.25) (width 0.8) (layer F.Cu) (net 12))
 (segment (start 4.5 -8) (end 5.5 -7) (width 0.8) (layer F.Cu) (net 12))
 (segment (start 10.25 -11) (end 10.75 -10.5) (width 0.25) (layer F.Cu) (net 12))
 (segment (start 5 -11) (end 10.25 -11) (width 0.25) (layer F.Cu) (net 12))
 (via (at 10.75 -10.5) (size 0.8) (drill 0.4) (layers F.Cu B.Cu) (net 12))
 (segment (start 5.5 -7) (end 5.5 -3.25) (width 0.8) (layer B.Cu) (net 12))
 (segment (start 4.5 -8) (end 5.5 -7) (width 0.8) (layer B.Cu) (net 12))
 (segment (start 4.5 -9.005) (end 4.5 -8) (width 0.8) (layer B.Cu) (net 12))
 (segment (start 10.75 -10.5) (end 10.25 -11) (width 0.25) (layer B.Cu) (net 12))
 (segment (start 10.25 -11) (end 5 -11) (width 0.25) (layer B.Cu) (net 12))
 (segment (start 5 -11) (end 4.5 -10.5) (width 0.25) (layer B.Cu) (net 12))
 (segment (start 4.5 -10.5) (end 4.5 -9.005) (width 0.25) (layer B.Cu) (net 12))
 (segment (start 10.85 -10.6) (end 10.75 -10.5) (width 1.5) (layer F.Cu) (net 12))
 (segment (start 12.2625 -10.6) (end 10.85 -10.6) (width 1.5) (layer F.Cu) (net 12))
 (segment (start -1.75 8.75) (end -1.75 9.25) (width 0.8) (layer F.Cu) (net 5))
 (segment (start 6.75 8.75) (end 6.75 7.25) (width 0.8) (layer B.Cu) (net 5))
 (segment (start 6.75 7.25) (end 6.5 7) (width 0.8) (layer B.Cu) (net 5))
 (segment (start 6.5 7) (end 2.25 7) (width 0.8) (layer B.Cu) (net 5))
 (segment (start 2.25 7) (end 0.75 8.5) (width 0.8) (layer B.Cu) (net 5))
 (segment (start -1.5 8.5) (end -1.75 8.75) (width 0.8) (layer B.Cu) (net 5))
 (segment (start 0.75 8.5) (end -1.5 8.5) (width 0.8) (layer B.Cu) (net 5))
 (segment (start 7.75 3) (end 6.75 4) (width 0.8) (layer B.Cu) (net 5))
 (segment (start 6.75 4) (end 6.75 8.75) (width 0.8) (layer B.Cu) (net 5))
 (segment (start 7.75 3) (end 7.5 3) (width 0.8) (layer F.Cu) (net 5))
 (segment (start -1.75 8.5) (end 0.75 8.5) (width 0.8) (layer F.Cu) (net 5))
 (segment (start 2.25 7) (end 6.5 7) (width 0.8) (layer F.Cu) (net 5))
 (segment (start 0.75 8.5) (end 2.25 7) (width 0.8) (layer F.Cu) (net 5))
 (segment (start 6.75 4) (end 6.75 8.75) (width 0.8) (layer F.Cu) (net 5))
 (segment (start 7.75 3) (end 6.75 4) (width 0.8) (layer F.Cu) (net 5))
 (segment (start 6.75 8.75) (end 8.75 8.75) (width 0.8) (layer F.Cu) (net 5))
 (segment (start 9 8.5) (end 10.5 8.5) (width 0.8) (layer F.Cu) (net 5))
 (segment (start 8.75 8.75) (end 9 8.5) (width 0.8) (layer F.Cu) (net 5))
 (segment (start 10.5 8.5) (end 10.5 8.5) (width 1.5) (layer F.Cu) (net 5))
 (via (at 10.5 8.5) (size 0.8) (drill 0.4) (layers F.Cu B.Cu) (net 5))
 (segment (start 10.5 8.5) (end 9 8.5) (width 0.25) (layer B.Cu) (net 5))
 (segment (start 9 8.5) (end 8.75 8.75) (width 0.25) (layer B.Cu) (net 5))
 (segment (start 8.75 8.75) (end 6.75 8.75) (width 0.25) (layer B.Cu) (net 5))
 (segment (start 11 8) (end 10.5 8.5) (width 1.5) (layer F.Cu) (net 5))
 (segment (start 12.2 8) (end 11 8) (width 1.5) (layer F.Cu) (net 5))
 (segment (start -13.67 -8.205001) (end -13.620001 -8.205001) (width 0.25) (layer F.Cu) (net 9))
 (segment (start -13.67 -0.364998) (end -13.7 -0.334998) (width 2) (layer F.Cu) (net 9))
 (segment (start -13.7 -8.175001) (end -13.67 -8.205001) (width 3.25) (layer F.Cu) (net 9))
 (segment (start -13.7 -0.334998) (end -13.7 -8.175001) (width 3.25) (layer F.Cu) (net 9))
 (via (at 10.668 -4.1148) (size 0.8) (drill 0.4) (layers F.Cu B.Cu) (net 9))
 (segment (start -13.67 -8.304999) (end -13.67 -0.364998) (width 3.25) (layer B.Cu) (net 9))
 (segment (start 8 -1.25) (end 10.668 -4.1148) (width 0.25) (layer F.Cu) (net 9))
 (segment (start 2.25 -1.25) (end 8 -1.25) (width 0.25) (layer F.Cu) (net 9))
 (segment (start 1.75 -1.75) (end 2.25 -1.25) (width 0.25) (layer F.Cu) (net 9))
 (segment (start 1.75 -11) (end 1.75 -1.75) (width 0.25) (layer F.Cu) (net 9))
 (segment (start 1 -11.5) (end 1.75 -11) (width 0.25) (layer F.Cu) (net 9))
 (segment (start -11.5 -11.5) (end 1 -11.5) (width 0.25) (layer F.Cu) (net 9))
 (segment (start -13.67 -9.33) (end -11.5 -11.5) (width 0.25) (layer F.Cu) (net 9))
 (segment (start -13.67 -8.304999) (end -13.67 -9.33) (width 0.25) (layer F.Cu) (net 9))
 (segment (start 10.6828 -4.1) (end 10.668 -4.1148) (width 0.8) (layer F.Cu) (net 9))
 (segment (start 12.2625 -4.1) (end 10.6828 -4.1) (width 1.5) (layer F.Cu) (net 9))
 (segment (start 8 -1.25) (end 10.668 -4.1148) (width 0.25) (layer B.Cu) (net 9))
 (segment (start 1.75 -1.75) (end 2.25 -1.25) (width 0.25) (layer B.Cu) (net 9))
 (segment (start 10.668 -4.1148) (end 10.75 -4.25) (width 0.25) (layer B.Cu) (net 9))
 (segment (start 1.75 -11) (end 1.75 -1.75) (width 0.25) (layer B.Cu) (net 9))
 (segment (start 2.25 -1.25) (end 8 -1.25) (width 0.25) (layer B.Cu) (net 9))
 (segment (start 1 -11.5) (end 1.75 -11) (width 0.25) (layer B.Cu) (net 9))
 (segment (start -11.5 -11.5) (end 1 -11.5) (width 0.25) (layer B.Cu) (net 9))
 (segment (start -13.67 -9.33) (end -11.5 -11.5) (width 0.25) (layer B.Cu) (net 9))
 (segment (start -13.67 -8.304999) (end -13.67 -9.33) (width 0.25) (layer B.Cu) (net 9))
 (segment (start -10.25 -8.25) (end -10.25 -0.309999) (width 3.25) (layer B.Cu) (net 1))
 (segment (start -10.17 -8.915) (end -10.17 -8.205001) (width 0.8) (layer F.Cu) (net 1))
 (segment (start -10.2 -8.175001) (end -10.17 -8.205001) (width 2) (layer F.Cu) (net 1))
 (segment (start -10.25 -0.409997) (end -10.25 -8.25) (width 3.25) (layer F.Cu) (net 1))
 (segment (start -10.17 -8.304999) (end -10.17 -8.33) (width 0.25) (layer F.Cu) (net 1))
 (via (at 10.668 -1.524) (size 0.8) (drill 0.4) (layers F.Cu B.Cu) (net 1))
 (segment (start 9 -0.5) (end 10.668 -1.524) (width 0.25) (layer F.Cu) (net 1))
 (segment (start 1 -10.75) (end 1 -1) (width 0.25) (layer F.Cu) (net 1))
 (segment (start 1.5 -0.5) (end 9 -0.5) (width 0.25) (layer F.Cu) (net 1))
 (segment (start 0.75 -11) (end 1 -10.75) (width 0.25) (layer F.Cu) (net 1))
 (segment (start -7.75 -11) (end 0.75 -11) (width 0.25) (layer F.Cu) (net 1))
 (segment (start 1 -1) (end 1.5 -0.5) (width 0.25) (layer F.Cu) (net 1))
 (segment (start -10.17 -8.58) (end -7.75 -11) (width 0.25) (layer F.Cu) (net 1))
 (segment (start -10.17 -8.304999) (end -10.17 -8.58) (width 0.25) (layer F.Cu) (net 1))
 (segment (start 10.692 -1.5) (end 10.668 -1.524) (width 0.8) (layer F.Cu) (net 1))
 (segment (start 12.175 -1.5) (end 10.692 -1.5) (width 1.5) (layer F.Cu) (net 1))
 (segment (start 9 -0.5) (end 10.668 -1.524) (width 0.25) (layer B.Cu) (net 1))
 (segment (start 1 -1) (end 1.5 -0.5) (width 0.25) (layer B.Cu) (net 1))
 (segment (start 1 -10.75) (end 1 -1) (width 0.25) (layer B.Cu) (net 1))
 (segment (start 1.5 -0.5) (end 9 -0.5) (width 0.25) (layer B.Cu) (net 1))
 (segment (start 0.75 -11) (end 1 -10.75) (width 0.25) (layer B.Cu) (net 1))
 (segment (start -7.75 -11) (end 0.75 -11) (width 0.25) (layer B.Cu) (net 1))
 (segment (start -10.17 -8.58) (end -7.75 -11) (width 0.25) (layer B.Cu) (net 1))
 (segment (start -10.17 -8.304999) (end -10.17 -8.58) (width 0.25) (layer B.Cu) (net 1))
 (segment (start -14.83 5.3984) (end -14.83 8.984) (width 0.8) (layer B.Cu) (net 17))
 (segment (start -14.83 5.3984) (end -14.83 8.984) (width 0.8) (layer F.Cu) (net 17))
 (segment (start -19 3.105) (end -19.16 3.265) (width 0.8) (layer F.Cu) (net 15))
 (segment (start -19 3.355) (end -19.16 3.515) (width 0.8) (layer F.Cu) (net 15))
 (segment (start -19 -2.285) (end -19 3.355) (width 0.8) (layer F.Cu) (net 15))
 (segment (start -19 3.355) (end -19.16 3.515) (width 0.8) (layer B.Cu) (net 15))
 (segment (start -19 -2.285) (end -19 3.355) (width 0.8) (layer B.Cu) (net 15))
 (segment (start -21.5 3.065) (end -21.7 3.265) (width 0.8) (layer F.Cu) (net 16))
 (segment (start -21.5 3.315) (end -21.7 3.515) (width 0.8) (layer F.Cu) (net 16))
 (segment (start -21.5 -2.285) (end -21.5 3.315) (width 0.8) (layer F.Cu) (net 16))
 (segment (start -21.5 3.315) (end -21.7 3.515) (width 0.8) (layer B.Cu) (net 16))
 (segment (start -21.5 -2.285) (end -21.5 3.315) (width 0.8) (layer B.Cu) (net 16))
 (segment (start 15.2375 1.5625) (end 15.3 1.5) (width 0.8) (layer F.Cu) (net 4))
 (segment (start 15.3 4.0375) (end 15.2375 4.1) (width 1.5) (layer F.Cu) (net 4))
 (segment (start 15.3 1.5) (end 15.3 4.0375) (width 1.5) (layer F.Cu) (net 4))
 (segment (start 15.275 -4.0625) (end 15.2375 -4.1) (width 0.8) (layer F.Cu) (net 2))
 (segment (start 15.2375 -1.5375) (end 15.275 -1.5) (width 1.5) (layer F.Cu) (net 2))
 (segment (start 15.2375 -4.1) (end 15.2375 -1.5375) (width 1.5) (layer F.Cu) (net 2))
 (segment (start 15.2125 -8.1625) (end 15.325 -8.05) (width 0.8) (layer F.Cu) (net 7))
 (segment (start 15.2375 -8.0625) (end 15.3 -8) (width 1.5) (layer F.Cu) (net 7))
 (segment (start 15.2375 -10.6) (end 15.2375 -8.0625) (width 1.5) (layer F.Cu) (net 7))
 (segment (start -6 3.04) (end -2.25 3.04) (width 0.8) (layer F.Cu) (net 13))
 (segment (start -6 3.04) (end -2.25 3.04) (width 0.8) (layer B.Cu) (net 13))
 (segment (start -6 0.5) (end -2.25 0.5) (width 0.8) (layer F.Cu) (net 14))
 (segment (start -6 0.5) (end -2.25 0.5) (width 0.8) (layer B.Cu) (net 14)))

